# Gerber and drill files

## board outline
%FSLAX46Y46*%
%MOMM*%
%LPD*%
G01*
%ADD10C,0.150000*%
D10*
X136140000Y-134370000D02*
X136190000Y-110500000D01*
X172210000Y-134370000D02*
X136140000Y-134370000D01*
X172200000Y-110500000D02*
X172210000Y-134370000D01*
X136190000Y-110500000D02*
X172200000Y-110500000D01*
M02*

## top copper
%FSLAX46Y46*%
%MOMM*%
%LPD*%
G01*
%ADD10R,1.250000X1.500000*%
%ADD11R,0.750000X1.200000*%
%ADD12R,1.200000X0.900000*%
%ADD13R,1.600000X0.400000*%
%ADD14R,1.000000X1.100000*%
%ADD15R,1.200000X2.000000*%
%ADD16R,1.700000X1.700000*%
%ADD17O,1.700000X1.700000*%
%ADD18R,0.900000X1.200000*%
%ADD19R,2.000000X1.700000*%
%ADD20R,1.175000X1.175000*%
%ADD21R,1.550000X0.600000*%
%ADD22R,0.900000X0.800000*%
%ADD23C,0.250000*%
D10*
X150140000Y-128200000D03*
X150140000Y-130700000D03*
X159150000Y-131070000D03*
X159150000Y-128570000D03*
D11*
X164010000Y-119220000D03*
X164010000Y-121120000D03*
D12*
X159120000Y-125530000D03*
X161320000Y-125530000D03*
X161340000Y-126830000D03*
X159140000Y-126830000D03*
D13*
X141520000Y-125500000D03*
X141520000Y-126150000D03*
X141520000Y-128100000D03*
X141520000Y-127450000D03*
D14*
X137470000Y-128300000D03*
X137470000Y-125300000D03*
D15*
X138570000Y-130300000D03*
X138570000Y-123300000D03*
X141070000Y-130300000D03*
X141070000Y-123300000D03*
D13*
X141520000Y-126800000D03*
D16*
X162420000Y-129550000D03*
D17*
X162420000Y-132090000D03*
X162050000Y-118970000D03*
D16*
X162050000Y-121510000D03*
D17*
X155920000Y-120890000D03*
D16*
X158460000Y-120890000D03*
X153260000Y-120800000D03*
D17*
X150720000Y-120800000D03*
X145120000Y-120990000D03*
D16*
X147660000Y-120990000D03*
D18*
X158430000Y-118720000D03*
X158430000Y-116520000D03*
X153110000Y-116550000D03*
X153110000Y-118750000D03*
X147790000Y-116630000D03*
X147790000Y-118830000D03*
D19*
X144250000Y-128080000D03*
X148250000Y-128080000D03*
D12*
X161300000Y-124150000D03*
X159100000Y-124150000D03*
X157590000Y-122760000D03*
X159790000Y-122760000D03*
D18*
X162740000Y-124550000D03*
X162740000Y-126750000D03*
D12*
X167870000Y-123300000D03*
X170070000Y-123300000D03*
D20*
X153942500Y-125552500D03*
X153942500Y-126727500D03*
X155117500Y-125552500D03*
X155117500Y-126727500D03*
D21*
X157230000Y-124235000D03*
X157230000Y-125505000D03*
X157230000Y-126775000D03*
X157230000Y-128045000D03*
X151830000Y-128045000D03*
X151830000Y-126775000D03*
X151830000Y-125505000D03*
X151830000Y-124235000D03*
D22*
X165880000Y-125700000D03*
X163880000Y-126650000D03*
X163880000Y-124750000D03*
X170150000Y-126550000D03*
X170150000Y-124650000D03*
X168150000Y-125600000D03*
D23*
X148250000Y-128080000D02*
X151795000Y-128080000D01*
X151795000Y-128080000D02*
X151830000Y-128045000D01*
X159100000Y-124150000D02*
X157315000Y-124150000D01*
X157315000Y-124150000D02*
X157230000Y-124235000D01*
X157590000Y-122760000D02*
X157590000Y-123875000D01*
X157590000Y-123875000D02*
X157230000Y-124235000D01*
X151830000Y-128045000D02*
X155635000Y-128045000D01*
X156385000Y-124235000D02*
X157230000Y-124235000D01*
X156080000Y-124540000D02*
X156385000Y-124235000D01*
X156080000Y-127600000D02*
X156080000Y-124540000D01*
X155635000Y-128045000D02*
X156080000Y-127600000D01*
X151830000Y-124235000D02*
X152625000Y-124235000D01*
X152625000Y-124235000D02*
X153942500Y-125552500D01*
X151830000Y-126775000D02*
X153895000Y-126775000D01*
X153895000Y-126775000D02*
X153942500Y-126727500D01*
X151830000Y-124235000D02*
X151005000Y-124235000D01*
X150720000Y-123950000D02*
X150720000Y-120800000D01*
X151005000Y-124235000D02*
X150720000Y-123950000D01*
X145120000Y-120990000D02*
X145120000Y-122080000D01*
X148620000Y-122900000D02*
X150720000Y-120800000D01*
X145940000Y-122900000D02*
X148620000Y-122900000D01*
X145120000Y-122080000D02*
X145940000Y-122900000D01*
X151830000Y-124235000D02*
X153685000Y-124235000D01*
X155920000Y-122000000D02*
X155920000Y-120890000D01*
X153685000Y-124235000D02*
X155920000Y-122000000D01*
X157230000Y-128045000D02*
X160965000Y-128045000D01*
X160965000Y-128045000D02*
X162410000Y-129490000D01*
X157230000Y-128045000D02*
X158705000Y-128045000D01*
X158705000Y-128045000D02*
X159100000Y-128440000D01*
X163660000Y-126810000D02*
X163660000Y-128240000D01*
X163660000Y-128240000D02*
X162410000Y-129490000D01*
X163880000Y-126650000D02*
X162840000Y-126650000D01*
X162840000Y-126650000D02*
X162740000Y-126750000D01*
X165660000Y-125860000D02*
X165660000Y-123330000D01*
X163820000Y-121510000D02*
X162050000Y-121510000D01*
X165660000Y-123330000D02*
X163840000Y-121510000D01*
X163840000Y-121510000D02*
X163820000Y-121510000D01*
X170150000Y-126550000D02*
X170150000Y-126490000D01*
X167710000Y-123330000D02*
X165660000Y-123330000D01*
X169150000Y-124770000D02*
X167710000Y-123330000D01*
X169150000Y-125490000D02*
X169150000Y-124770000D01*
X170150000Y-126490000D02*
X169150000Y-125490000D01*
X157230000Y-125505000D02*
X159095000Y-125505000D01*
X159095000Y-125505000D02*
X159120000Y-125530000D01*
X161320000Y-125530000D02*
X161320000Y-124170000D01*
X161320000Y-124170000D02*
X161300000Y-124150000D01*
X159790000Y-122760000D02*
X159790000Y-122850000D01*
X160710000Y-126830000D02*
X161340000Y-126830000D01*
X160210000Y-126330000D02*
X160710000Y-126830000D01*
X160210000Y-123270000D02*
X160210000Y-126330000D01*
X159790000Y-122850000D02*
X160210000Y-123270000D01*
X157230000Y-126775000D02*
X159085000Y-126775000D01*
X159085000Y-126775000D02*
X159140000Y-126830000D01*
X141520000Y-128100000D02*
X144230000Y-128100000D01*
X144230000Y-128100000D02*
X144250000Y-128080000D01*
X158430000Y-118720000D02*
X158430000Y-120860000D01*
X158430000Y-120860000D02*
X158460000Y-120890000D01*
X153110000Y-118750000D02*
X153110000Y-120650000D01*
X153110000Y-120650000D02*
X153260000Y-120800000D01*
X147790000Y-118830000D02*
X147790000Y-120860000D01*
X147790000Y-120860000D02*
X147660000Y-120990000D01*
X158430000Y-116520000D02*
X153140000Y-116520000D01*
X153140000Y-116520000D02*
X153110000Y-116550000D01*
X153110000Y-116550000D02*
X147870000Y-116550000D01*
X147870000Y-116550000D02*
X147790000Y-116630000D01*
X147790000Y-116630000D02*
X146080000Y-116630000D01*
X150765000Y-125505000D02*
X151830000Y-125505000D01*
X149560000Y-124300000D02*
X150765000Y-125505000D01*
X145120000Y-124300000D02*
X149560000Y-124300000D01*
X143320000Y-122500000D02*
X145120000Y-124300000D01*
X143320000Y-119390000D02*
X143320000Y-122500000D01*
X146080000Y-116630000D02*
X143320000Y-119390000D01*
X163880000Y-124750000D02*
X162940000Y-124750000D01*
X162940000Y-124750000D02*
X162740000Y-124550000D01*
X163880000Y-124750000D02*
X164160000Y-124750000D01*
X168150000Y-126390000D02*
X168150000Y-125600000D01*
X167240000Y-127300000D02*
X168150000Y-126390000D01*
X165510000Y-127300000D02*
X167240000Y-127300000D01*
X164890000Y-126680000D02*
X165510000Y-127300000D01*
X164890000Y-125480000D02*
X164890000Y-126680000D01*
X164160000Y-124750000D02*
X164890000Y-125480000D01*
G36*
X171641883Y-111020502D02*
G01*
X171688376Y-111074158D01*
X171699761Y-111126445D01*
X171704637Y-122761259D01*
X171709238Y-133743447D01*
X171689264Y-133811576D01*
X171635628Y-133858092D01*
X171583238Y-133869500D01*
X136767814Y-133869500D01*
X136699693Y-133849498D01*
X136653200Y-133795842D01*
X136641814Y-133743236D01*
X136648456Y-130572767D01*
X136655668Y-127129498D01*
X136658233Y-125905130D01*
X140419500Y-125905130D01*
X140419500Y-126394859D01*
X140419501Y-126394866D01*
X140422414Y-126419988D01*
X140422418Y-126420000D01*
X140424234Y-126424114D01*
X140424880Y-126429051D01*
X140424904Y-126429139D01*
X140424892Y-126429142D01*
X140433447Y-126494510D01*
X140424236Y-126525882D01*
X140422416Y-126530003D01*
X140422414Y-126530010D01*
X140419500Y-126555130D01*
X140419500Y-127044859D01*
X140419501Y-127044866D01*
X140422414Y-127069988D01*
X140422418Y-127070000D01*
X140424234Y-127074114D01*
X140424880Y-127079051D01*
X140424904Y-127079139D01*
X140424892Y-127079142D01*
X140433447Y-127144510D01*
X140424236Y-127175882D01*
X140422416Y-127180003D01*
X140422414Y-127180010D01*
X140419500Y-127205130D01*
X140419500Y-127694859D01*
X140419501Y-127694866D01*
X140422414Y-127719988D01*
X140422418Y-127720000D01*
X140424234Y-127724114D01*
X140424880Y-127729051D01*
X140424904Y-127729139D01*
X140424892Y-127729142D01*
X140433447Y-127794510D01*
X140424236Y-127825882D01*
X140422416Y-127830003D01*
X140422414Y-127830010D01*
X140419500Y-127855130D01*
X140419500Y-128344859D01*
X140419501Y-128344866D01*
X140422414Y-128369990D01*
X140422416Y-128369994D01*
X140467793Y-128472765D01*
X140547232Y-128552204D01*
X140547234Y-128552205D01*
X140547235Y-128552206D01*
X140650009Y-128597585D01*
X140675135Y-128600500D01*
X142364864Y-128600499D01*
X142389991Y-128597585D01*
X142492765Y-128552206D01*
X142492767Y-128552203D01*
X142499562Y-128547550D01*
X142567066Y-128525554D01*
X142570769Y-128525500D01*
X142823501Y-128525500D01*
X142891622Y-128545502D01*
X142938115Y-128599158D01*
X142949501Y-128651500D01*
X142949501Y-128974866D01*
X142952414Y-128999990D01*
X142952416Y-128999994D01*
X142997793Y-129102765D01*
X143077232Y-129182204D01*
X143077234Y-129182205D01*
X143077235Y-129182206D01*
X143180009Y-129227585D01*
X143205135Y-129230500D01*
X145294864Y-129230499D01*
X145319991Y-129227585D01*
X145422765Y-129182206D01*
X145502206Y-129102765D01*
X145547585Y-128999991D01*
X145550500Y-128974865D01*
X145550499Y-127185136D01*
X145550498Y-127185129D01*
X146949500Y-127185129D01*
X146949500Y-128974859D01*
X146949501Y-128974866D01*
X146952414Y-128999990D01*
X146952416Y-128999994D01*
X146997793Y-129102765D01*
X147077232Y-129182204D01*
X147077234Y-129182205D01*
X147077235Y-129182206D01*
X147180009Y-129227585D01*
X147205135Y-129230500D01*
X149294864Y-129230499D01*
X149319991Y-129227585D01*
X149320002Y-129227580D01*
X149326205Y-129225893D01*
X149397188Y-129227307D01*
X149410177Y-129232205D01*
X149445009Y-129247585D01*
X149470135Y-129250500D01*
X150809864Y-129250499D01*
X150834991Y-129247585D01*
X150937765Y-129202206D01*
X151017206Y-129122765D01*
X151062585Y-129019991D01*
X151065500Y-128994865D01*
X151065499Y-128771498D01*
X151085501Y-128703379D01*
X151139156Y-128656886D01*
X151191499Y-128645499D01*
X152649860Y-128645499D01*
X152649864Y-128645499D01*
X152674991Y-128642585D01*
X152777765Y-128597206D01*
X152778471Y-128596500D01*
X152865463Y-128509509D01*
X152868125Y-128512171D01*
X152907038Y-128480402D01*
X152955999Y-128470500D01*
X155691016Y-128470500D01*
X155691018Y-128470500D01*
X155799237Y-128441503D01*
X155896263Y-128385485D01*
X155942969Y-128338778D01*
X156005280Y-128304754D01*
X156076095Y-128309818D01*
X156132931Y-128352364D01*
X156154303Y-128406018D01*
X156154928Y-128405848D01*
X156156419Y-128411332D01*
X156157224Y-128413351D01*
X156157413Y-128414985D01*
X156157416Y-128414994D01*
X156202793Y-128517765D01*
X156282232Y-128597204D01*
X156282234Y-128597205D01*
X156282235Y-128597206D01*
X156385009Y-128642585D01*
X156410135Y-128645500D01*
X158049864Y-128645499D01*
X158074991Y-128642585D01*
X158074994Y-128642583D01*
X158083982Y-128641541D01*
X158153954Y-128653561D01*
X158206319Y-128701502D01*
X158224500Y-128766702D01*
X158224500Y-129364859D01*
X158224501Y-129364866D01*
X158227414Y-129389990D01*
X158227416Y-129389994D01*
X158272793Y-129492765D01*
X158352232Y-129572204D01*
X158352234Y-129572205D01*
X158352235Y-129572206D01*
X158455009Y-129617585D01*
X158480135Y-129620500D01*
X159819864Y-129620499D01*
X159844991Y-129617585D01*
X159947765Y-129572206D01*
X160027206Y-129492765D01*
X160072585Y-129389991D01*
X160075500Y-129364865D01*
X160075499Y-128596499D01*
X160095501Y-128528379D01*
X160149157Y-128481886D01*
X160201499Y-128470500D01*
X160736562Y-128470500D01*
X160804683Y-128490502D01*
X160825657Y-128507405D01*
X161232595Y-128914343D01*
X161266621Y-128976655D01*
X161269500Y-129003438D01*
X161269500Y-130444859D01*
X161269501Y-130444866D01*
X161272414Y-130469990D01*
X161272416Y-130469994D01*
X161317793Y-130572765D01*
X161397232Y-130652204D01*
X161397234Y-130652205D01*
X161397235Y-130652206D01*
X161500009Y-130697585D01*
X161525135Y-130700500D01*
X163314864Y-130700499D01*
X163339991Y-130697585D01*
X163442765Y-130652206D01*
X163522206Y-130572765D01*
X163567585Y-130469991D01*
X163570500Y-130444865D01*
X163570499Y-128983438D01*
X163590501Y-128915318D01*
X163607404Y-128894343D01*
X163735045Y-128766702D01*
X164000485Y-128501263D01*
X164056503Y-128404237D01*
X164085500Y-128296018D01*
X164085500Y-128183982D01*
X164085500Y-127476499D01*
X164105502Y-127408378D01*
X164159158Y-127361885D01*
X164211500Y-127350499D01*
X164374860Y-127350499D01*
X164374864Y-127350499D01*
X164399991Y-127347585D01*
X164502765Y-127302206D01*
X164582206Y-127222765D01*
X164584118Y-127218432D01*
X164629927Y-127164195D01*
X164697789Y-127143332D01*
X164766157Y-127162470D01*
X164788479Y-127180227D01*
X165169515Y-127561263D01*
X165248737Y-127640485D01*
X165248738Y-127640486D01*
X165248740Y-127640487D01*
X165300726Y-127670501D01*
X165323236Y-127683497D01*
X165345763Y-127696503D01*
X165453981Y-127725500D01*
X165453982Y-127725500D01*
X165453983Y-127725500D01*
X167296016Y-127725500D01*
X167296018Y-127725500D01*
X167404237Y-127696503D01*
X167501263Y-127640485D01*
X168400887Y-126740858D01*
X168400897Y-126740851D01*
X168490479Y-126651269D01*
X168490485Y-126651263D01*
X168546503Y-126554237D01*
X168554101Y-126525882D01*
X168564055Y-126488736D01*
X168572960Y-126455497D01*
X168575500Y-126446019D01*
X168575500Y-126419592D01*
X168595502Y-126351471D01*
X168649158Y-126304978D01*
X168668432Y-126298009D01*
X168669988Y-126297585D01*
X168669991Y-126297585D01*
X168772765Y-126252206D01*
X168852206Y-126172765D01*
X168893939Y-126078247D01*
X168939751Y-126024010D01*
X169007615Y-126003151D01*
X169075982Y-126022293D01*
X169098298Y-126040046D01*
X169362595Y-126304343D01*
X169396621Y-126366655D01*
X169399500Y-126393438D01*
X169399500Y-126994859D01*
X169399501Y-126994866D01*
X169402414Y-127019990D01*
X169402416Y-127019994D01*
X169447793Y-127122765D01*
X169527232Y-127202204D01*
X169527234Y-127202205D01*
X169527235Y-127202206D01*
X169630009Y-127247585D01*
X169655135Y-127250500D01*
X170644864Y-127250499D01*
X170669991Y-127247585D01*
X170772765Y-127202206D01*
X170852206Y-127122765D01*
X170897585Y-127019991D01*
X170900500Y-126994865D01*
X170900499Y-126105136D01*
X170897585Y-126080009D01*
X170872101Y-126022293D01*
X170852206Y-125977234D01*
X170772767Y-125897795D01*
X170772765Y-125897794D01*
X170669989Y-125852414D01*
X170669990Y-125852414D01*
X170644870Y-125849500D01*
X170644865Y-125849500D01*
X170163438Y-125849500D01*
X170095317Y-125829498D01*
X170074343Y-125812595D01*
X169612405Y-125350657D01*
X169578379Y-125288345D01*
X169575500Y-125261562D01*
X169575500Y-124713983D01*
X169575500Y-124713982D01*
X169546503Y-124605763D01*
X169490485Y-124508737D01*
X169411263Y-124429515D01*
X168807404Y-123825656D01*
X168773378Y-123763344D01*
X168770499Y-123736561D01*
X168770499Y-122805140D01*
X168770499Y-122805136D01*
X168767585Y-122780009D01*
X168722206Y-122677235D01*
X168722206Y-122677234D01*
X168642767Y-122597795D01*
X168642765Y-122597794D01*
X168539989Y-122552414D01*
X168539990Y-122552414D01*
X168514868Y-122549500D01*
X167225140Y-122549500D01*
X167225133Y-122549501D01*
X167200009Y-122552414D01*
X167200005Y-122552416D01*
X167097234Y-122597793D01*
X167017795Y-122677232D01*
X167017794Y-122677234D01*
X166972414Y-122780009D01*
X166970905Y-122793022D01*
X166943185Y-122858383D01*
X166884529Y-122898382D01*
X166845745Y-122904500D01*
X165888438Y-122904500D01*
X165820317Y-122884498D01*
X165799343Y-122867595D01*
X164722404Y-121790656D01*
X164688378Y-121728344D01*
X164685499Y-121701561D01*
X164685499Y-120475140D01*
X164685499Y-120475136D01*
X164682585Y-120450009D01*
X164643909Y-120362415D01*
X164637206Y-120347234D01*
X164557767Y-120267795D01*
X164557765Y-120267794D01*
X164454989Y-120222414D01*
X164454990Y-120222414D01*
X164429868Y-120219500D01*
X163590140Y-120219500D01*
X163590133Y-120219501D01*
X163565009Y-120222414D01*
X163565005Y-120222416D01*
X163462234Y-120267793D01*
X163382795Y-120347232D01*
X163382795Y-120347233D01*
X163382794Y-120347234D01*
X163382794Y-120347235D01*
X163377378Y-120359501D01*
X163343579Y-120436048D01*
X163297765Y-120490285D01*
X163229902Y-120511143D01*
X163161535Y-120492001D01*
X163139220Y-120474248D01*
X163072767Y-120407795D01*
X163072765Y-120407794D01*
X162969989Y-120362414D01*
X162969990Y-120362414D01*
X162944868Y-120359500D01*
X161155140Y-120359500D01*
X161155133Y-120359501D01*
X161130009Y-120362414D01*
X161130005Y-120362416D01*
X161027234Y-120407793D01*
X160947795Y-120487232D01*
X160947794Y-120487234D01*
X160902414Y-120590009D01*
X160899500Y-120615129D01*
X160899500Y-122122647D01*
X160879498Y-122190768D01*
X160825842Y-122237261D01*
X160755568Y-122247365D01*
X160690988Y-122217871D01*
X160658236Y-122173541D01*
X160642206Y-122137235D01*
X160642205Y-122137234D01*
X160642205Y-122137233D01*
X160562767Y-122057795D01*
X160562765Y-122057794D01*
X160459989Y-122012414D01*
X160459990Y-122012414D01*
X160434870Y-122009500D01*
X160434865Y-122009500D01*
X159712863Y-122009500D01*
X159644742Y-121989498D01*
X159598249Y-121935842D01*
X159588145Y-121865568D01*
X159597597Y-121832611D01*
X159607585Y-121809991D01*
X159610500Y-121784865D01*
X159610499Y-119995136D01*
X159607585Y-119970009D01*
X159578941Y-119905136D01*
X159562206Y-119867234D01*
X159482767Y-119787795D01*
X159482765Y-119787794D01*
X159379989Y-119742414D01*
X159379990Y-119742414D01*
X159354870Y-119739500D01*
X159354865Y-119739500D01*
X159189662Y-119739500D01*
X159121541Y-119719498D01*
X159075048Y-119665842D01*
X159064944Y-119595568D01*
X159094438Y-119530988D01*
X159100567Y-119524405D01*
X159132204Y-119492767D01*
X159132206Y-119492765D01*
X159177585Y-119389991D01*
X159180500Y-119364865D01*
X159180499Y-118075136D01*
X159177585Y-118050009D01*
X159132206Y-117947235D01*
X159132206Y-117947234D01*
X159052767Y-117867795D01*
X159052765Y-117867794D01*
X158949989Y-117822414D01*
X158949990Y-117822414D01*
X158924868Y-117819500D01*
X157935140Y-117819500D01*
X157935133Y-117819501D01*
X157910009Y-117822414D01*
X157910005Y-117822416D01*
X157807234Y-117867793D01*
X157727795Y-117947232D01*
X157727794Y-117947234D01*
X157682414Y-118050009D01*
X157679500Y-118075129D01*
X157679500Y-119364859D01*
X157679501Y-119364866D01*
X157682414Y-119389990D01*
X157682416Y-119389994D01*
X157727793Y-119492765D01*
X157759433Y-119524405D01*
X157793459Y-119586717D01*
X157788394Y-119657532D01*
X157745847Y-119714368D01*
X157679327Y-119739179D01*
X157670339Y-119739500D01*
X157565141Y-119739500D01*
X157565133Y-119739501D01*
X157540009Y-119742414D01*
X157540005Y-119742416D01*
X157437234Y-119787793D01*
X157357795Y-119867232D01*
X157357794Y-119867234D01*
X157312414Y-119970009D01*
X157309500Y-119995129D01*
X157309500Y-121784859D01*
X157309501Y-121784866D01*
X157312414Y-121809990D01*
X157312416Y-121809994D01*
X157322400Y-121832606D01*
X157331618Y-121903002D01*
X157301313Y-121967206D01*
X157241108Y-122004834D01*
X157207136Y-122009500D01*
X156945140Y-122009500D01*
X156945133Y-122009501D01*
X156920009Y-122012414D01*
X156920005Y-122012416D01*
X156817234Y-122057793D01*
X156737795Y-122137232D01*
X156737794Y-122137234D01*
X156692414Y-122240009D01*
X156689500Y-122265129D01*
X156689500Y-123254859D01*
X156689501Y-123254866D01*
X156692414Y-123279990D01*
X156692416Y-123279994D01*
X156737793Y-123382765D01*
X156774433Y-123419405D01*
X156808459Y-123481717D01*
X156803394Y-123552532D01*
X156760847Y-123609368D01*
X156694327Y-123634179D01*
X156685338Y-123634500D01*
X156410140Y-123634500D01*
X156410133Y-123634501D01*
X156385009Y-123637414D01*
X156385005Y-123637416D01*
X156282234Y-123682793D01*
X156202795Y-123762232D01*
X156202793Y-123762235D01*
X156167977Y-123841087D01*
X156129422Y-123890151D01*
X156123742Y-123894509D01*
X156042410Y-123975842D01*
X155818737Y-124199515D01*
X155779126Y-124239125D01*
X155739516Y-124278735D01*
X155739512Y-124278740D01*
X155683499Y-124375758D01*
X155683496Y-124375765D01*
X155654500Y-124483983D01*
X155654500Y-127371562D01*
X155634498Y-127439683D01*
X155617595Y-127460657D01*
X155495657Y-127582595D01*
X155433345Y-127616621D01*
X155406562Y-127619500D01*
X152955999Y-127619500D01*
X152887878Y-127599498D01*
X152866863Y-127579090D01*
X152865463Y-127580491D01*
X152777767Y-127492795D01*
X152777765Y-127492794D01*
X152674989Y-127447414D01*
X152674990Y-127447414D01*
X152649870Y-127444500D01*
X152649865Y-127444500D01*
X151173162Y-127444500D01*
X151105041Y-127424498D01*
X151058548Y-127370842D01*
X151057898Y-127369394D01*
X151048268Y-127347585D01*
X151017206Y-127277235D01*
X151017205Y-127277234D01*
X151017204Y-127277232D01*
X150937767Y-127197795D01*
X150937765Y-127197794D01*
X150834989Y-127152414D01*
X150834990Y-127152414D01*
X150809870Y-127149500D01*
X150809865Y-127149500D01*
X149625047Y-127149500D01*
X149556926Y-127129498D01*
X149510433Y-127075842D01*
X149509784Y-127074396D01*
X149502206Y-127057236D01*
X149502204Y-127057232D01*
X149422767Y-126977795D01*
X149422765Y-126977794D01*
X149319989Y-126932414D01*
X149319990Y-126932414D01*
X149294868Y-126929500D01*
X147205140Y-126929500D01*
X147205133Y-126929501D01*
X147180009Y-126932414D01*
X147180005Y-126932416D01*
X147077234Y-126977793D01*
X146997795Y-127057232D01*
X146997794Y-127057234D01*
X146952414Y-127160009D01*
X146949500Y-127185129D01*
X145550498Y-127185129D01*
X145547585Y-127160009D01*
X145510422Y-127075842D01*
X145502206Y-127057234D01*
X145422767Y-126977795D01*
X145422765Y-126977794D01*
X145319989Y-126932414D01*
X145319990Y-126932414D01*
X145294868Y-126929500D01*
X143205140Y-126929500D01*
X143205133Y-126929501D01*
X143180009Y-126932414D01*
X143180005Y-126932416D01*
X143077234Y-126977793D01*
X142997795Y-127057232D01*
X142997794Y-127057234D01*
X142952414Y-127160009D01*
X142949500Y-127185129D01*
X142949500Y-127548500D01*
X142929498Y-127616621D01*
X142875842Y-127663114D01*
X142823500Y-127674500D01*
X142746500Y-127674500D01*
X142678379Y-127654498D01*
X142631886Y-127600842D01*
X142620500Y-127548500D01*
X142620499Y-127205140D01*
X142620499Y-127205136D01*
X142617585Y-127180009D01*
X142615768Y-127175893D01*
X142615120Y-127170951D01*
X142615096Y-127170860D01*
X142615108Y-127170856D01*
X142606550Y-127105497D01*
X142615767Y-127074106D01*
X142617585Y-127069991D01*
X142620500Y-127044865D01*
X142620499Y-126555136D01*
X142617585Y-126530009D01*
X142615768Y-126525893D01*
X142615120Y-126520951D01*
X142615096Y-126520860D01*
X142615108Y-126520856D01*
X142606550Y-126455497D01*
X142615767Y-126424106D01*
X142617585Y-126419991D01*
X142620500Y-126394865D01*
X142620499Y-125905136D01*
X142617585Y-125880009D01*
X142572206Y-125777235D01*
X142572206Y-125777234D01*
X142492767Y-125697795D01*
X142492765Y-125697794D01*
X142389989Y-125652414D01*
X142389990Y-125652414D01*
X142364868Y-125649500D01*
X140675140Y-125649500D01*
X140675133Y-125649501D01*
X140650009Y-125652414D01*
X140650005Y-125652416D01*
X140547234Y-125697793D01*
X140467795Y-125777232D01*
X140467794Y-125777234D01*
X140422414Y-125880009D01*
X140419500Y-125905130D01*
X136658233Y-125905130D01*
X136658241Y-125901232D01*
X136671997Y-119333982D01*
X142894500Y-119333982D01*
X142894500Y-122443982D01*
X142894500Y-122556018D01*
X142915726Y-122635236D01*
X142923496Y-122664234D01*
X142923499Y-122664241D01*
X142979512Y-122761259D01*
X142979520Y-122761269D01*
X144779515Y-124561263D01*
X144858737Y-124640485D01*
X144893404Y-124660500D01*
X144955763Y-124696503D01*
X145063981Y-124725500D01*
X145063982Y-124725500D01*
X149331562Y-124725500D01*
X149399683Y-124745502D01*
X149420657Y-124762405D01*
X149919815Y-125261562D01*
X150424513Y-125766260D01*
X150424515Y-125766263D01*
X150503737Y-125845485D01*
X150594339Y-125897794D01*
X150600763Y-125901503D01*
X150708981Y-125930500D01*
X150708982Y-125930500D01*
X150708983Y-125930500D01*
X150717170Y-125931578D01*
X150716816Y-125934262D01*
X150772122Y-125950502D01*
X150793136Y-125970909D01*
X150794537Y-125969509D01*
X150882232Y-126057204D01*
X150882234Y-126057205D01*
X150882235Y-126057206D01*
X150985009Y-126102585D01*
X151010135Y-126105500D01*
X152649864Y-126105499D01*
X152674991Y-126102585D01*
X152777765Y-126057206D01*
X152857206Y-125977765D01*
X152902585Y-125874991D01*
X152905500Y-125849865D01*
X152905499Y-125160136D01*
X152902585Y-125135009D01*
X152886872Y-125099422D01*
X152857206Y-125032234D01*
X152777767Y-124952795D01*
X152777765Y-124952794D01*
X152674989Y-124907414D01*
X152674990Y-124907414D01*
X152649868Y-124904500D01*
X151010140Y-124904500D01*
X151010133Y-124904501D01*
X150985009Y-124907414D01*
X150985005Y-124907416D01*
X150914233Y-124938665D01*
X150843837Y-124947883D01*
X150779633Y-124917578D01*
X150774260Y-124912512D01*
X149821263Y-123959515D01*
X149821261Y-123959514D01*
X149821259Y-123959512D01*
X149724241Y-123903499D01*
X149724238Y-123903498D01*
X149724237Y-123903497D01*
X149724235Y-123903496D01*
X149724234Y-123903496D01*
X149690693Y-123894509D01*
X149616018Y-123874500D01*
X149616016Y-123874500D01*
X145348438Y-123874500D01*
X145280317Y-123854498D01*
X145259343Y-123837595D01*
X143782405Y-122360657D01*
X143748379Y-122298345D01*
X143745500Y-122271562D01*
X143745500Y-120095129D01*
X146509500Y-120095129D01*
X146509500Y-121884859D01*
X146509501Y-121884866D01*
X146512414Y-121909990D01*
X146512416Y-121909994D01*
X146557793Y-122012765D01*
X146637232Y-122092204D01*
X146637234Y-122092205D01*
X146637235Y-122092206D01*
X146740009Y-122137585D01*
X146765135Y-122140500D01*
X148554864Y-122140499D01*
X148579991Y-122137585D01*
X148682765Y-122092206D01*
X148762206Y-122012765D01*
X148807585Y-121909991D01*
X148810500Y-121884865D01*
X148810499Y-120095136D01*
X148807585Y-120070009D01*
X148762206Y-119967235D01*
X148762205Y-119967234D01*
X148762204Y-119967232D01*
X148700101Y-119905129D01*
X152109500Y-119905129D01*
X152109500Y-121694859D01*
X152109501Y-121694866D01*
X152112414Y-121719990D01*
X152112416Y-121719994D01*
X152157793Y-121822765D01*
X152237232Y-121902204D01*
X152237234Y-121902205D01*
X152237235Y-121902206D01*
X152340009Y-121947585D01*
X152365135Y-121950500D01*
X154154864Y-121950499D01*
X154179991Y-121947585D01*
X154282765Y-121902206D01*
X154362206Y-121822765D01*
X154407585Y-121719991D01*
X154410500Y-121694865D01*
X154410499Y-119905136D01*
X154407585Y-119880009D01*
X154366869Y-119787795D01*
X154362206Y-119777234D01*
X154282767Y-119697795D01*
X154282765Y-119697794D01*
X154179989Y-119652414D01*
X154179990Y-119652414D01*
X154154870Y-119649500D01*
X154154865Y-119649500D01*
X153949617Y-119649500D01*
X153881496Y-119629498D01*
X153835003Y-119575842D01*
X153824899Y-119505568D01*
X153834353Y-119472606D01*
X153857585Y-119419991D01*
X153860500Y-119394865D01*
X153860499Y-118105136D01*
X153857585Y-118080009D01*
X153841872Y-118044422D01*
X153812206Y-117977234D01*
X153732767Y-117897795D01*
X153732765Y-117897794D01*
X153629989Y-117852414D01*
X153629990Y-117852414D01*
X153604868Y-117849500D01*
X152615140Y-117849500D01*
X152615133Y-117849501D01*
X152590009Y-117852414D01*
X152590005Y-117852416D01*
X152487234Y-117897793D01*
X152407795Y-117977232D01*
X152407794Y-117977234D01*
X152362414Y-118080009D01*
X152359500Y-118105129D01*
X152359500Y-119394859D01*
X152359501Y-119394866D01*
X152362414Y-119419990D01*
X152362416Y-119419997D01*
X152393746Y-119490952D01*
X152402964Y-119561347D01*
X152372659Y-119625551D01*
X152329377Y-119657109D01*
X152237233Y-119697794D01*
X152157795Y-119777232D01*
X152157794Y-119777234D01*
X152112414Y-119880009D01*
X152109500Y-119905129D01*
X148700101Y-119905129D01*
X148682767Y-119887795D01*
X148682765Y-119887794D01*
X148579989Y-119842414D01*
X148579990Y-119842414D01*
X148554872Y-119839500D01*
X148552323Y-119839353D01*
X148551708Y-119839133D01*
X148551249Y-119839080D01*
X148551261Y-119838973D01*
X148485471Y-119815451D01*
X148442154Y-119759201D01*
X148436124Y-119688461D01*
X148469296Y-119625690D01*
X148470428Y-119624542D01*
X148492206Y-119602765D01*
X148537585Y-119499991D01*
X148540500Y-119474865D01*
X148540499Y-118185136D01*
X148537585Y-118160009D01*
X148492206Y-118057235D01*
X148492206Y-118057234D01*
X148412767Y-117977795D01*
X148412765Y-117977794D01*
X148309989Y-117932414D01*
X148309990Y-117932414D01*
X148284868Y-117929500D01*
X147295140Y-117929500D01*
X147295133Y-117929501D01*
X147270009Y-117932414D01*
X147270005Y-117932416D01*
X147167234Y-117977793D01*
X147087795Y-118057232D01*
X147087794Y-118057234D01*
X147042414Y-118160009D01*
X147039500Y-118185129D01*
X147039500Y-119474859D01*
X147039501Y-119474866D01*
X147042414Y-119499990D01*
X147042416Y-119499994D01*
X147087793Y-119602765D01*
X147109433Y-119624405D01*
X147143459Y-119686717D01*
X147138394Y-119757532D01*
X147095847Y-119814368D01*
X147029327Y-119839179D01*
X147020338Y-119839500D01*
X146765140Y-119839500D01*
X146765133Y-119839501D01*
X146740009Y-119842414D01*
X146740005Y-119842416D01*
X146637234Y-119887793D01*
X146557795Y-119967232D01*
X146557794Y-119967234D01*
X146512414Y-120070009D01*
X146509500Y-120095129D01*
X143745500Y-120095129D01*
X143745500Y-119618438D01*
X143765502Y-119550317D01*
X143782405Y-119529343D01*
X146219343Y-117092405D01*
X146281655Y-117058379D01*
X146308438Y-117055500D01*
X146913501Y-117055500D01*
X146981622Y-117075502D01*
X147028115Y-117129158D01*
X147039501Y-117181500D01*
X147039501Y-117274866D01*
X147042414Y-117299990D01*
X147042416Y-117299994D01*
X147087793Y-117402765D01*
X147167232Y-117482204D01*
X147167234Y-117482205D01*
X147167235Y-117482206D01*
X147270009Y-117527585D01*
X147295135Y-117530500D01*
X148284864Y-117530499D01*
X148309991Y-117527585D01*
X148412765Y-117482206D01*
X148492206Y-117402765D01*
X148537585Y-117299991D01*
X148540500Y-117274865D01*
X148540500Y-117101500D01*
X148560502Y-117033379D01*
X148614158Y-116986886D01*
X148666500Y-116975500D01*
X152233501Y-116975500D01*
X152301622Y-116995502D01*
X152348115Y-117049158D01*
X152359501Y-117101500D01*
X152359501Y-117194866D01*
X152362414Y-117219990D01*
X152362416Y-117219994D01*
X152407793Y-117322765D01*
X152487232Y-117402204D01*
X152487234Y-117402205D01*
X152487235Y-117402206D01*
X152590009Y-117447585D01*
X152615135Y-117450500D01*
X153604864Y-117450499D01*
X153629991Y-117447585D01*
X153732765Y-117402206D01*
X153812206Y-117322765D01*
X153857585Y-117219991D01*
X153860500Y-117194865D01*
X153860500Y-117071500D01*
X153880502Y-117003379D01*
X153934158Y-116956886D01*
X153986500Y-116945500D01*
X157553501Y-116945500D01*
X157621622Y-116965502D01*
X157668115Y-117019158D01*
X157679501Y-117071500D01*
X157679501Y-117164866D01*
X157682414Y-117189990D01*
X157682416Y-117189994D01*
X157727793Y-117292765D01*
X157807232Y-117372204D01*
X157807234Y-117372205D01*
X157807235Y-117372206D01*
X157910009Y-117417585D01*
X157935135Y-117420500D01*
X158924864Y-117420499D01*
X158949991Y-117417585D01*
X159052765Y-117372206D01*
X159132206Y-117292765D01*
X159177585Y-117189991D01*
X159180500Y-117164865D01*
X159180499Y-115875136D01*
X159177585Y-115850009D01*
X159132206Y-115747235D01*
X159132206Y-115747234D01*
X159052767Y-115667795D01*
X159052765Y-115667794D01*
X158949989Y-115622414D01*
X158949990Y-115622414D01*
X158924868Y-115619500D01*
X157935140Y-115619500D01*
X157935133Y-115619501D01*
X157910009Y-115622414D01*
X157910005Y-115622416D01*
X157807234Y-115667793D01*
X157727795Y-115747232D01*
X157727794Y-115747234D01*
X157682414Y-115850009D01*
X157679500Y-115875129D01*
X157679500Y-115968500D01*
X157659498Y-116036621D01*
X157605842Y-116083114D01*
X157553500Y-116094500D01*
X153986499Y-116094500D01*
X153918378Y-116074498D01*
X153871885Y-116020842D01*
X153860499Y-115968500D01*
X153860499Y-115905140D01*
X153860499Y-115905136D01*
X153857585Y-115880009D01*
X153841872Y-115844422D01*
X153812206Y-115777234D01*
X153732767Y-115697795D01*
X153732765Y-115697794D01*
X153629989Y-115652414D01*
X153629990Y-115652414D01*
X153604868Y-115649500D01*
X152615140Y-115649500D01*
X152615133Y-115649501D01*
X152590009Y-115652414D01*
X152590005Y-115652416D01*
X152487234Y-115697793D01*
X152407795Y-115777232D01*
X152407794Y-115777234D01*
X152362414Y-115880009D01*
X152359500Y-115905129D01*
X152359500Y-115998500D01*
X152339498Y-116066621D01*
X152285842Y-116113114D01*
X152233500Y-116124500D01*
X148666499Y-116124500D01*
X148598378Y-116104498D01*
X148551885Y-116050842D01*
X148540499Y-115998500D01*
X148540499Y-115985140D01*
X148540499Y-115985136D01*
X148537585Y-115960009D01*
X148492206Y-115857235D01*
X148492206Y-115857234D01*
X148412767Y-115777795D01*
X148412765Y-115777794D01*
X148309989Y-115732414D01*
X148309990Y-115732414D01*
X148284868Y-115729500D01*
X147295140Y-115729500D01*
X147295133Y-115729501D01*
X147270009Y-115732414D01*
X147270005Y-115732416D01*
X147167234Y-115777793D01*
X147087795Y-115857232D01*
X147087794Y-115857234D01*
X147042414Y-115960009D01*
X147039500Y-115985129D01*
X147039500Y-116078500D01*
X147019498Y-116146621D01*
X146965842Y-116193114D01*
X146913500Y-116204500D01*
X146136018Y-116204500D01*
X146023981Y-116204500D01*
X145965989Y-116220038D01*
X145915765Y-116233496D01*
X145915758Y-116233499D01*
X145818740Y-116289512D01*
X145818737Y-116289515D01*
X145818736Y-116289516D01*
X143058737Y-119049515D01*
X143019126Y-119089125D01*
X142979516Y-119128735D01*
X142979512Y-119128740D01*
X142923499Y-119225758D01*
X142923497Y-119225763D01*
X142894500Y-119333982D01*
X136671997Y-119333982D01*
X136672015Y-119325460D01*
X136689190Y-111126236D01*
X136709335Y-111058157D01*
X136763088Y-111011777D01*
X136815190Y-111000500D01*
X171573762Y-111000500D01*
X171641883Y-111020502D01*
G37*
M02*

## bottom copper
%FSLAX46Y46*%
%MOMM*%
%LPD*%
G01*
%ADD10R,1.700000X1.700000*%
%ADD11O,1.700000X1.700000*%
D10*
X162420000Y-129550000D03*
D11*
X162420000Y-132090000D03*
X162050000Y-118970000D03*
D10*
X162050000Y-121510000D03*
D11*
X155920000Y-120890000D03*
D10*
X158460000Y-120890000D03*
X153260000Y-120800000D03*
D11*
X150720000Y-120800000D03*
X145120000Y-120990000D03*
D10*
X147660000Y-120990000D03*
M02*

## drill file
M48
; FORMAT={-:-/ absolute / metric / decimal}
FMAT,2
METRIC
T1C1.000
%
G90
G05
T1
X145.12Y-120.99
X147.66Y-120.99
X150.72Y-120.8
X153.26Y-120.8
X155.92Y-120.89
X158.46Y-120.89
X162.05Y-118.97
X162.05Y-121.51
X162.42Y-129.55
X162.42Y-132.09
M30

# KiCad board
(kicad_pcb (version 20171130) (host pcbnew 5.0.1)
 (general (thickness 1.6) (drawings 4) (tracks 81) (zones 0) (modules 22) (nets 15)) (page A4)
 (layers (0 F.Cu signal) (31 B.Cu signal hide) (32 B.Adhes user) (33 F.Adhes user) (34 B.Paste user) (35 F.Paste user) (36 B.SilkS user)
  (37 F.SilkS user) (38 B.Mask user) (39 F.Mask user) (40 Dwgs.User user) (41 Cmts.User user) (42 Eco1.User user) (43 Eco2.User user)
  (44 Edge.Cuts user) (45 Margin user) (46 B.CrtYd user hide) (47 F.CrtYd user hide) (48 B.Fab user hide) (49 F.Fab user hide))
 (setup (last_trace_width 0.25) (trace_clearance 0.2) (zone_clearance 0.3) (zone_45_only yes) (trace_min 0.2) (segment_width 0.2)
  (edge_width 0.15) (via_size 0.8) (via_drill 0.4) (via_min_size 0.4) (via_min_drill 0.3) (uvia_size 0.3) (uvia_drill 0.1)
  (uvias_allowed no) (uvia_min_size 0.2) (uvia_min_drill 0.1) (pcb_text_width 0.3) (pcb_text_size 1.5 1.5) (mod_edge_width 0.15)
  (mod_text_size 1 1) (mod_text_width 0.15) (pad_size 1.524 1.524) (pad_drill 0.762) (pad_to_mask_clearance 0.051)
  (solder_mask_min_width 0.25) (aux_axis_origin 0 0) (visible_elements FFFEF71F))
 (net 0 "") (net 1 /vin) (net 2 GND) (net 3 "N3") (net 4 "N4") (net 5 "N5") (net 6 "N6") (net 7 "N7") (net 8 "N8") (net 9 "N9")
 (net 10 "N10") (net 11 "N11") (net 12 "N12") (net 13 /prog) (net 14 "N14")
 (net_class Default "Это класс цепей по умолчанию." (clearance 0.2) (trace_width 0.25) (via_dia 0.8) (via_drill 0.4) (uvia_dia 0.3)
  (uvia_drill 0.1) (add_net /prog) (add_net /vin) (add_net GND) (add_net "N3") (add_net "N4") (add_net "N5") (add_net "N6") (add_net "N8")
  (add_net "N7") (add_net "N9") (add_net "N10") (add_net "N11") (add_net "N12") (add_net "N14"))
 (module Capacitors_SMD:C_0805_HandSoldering (layer F.Cu) (at 150.14 129.45 270)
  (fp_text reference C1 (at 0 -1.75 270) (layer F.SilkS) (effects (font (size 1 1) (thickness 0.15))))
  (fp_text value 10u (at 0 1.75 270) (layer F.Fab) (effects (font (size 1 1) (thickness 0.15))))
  (pad 1 smd rect (at -1.25 0 270) (size 1.5 1.25) (layers F.Cu F.Paste F.Mask) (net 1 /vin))
  (pad 2 smd rect (at 1.25 0 270) (size 1.5 1.25) (layers F.Cu F.Paste F.Mask) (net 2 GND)))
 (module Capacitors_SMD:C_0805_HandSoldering (layer F.Cu) (at 159.15 129.82 270)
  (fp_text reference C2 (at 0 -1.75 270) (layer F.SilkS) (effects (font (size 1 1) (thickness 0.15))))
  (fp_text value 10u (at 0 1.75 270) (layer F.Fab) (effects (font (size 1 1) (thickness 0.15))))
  (pad 2 smd rect (at 1.25 0 270) (size 1.5 1.25) (layers F.Cu F.Paste F.Mask) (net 2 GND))
  (pad 1 smd rect (at -1.25 0 270) (size 1.5 1.25) (layers F.Cu F.Paste F.Mask) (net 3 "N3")))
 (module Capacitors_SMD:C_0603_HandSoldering (layer F.Cu) (at 164.01 120.17 90)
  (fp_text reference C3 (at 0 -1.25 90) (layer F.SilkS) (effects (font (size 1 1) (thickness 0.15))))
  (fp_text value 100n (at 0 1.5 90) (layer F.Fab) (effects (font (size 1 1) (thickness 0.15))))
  (pad 2 smd rect (at 0.95 0 90) (size 1.2 0.75) (layers F.Cu F.Paste F.Mask) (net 2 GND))
  (pad 1 smd rect (at -0.95 0 90) (size 1.2 0.75) (layers F.Cu F.Paste F.Mask) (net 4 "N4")))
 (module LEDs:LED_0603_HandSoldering (layer F.Cu) (at 160.22 125.53)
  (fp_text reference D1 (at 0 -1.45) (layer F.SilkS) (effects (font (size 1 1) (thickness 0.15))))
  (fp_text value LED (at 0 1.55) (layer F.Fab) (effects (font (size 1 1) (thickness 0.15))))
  (pad 1 smd rect (at -1.1 0) (size 1.2 0.9) (layers F.Cu F.Paste F.Mask) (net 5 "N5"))
  (pad 2 smd rect (at 1.1 0) (size 1.2 0.9) (layers F.Cu F.Paste F.Mask) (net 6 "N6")))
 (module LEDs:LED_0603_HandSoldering (layer F.Cu) (at 160.24 126.83)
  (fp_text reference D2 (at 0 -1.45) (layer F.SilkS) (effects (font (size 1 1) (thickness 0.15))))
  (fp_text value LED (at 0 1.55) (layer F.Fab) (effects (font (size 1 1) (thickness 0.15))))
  (pad 2 smd rect (at 1.1 0) (size 1.2 0.9) (layers F.Cu F.Paste F.Mask) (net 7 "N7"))
  (pad 1 smd rect (at -1.1 0) (size 1.2 0.9) (layers F.Cu F.Paste F.Mask) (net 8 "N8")))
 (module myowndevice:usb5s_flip (layer F.Cu) (at 142.42 126.8 270)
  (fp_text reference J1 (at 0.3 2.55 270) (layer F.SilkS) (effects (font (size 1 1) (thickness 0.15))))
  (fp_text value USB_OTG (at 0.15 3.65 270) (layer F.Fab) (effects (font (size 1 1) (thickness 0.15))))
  (pad 5 smd rect (at -1.3 0.9 270) (size 0.4 1.6) (layers F.Cu F.Paste F.Mask) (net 2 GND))
  (pad 4 smd rect (at -0.65 0.9 270) (size 0.4 1.6) (layers F.Cu F.Paste F.Mask))
  (pad 1 smd rect (at 1.3 0.9 270) (size 0.4 1.6) (layers F.Cu F.Paste F.Mask) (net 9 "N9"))
  (pad 2 smd rect (at 0.65 0.9 270) (size 0.4 1.6) (layers F.Cu F.Paste F.Mask))
  (pad 5 smd rect (at 1.5 4.95 270) (size 1.1 1) (layers F.Cu F.Paste F.Mask) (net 2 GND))
  (pad 5 smd rect (at -1.5 4.95 270) (size 1.1 1) (layers F.Cu F.Paste F.Mask) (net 2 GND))
  (pad 5 smd rect (at 3.5 3.85 270) (size 2 1.2) (layers F.Cu F.Paste F.Mask) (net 2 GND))
  (pad 5 smd rect (at -3.5 3.85 270) (size 2 1.2) (layers F.Cu F.Paste F.Mask) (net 2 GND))
  (pad 5 smd rect (at 3.5 1.35 270) (size 2 1.2) (layers F.Cu F.Paste F.Mask) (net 2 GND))
  (pad 5 smd rect (at -3.5 1.35 270) (size 2 1.2) (layers F.Cu F.Paste F.Mask) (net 2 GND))
  (pad 3 smd rect (at 0 0.9 270) (size 0.4 1.6) (layers F.Cu F.Paste F.Mask)))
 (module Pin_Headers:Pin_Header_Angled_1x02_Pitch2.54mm (layer B.Cu) (at 162.42 129.55 180)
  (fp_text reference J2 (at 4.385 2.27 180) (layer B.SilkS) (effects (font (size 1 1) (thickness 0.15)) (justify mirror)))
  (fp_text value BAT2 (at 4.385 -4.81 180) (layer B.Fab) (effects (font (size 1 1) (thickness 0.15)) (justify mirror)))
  (pad 1 thru_hole rect (at 0 0 180) (size 1.7 1.7) (drill 1) (layers *.Cu *.Mask) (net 3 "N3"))
  (pad 2 thru_hole oval (at 0 -2.54 180) (size 1.7 1.7) (drill 1) (layers *.Cu *.Mask) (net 2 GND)))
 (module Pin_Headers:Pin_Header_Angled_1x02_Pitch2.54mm (layer B.Cu) (at 162.05 121.51)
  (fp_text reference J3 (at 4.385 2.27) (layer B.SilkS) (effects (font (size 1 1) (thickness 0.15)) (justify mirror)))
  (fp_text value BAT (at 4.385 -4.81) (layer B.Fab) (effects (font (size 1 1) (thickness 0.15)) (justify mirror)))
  (pad 2 thru_hole oval (at 0 -2.54) (size 1.7 1.7) (drill 1) (layers *.Cu *.Mask) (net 2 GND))
  (pad 1 thru_hole rect (at 0 0) (size 1.7 1.7) (drill 1) (layers *.Cu *.Mask) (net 4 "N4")))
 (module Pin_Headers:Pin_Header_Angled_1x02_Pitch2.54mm (layer B.Cu) (at 158.46 120.89 90)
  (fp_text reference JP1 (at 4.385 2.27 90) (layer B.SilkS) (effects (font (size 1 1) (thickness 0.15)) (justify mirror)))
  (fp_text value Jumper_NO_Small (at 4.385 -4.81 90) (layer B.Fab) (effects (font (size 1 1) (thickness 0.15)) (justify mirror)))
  (pad 2 thru_hole oval (at 0 -2.54 90) (size 1.7 1.7) (drill 1) (layers *.Cu *.Mask) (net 2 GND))
  (pad 1 thru_hole rect (at 0 0 90) (size 1.7 1.7) (drill 1) (layers *.Cu *.Mask) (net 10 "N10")))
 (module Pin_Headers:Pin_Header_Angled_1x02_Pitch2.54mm (layer B.Cu) (at 153.26 120.8 90)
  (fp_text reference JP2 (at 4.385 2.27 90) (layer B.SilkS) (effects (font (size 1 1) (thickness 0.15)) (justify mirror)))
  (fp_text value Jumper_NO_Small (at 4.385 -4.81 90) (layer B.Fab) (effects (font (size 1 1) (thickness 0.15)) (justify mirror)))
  (pad 1 thru_hole rect (at 0 0 90) (size 1.7 1.7) (drill 1) (layers *.Cu *.Mask) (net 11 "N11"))
  (pad 2 thru_hole oval (at 0 -2.54 90) (size 1.7 1.7) (drill 1) (layers *.Cu *.Mask) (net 2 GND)))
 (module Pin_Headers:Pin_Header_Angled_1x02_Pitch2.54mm (layer B.Cu) (at 147.66 120.99 90)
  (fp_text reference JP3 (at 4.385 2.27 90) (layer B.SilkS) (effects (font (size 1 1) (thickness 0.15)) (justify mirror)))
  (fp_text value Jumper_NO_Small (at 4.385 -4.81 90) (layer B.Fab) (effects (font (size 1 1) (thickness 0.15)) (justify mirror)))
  (pad 2 thru_hole oval (at 0 -2.54 90) (size 1.7 1.7) (drill 1) (layers *.Cu *.Mask) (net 2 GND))
  (pad 1 thru_hole rect (at 0 0 90) (size 1.7 1.7) (drill 1) (layers *.Cu *.Mask) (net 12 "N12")))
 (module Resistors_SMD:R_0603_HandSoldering (layer F.Cu) (at 158.43 117.62 90)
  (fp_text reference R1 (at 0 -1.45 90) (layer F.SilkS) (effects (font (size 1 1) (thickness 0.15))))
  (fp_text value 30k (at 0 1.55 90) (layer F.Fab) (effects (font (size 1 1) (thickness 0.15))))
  (pad 1 smd rect (at -1.1 0 90) (size 1.2 0.9) (layers F.Cu F.Paste F.Mask) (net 10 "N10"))
  (pad 2 smd rect (at 1.1 0 90) (size 1.2 0.9) (layers F.Cu F.Paste F.Mask) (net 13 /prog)))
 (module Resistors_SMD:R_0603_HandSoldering (layer F.Cu) (at 153.11 117.65 90)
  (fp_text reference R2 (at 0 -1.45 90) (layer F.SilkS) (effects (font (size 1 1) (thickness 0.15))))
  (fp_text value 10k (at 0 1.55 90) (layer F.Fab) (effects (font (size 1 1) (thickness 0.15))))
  (pad 2 smd rect (at 1.1 0 90) (size 1.2 0.9) (layers F.Cu F.Paste F.Mask) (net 13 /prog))
  (pad 1 smd rect (at -1.1 0 90) (size 1.2 0.9) (layers F.Cu F.Paste F.Mask) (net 11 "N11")))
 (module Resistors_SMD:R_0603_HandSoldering (layer F.Cu) (at 147.79 117.73 90)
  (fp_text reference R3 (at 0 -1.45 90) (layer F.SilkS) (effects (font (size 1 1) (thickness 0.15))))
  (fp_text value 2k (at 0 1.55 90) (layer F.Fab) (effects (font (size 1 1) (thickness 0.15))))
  (pad 2 smd rect (at 1.1 0 90) (size 1.2 0.9) (layers F.Cu F.Paste F.Mask) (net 13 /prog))
  (pad 1 smd rect (at -1.1 0 90) (size 1.2 0.9) (layers F.Cu F.Paste F.Mask) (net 12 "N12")))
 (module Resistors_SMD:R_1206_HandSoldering (layer F.Cu) (at 146.25 128.08 180)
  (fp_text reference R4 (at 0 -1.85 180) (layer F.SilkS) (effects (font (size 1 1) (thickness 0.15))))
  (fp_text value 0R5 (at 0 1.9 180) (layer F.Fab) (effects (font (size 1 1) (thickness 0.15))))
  (pad 2 smd rect (at 2 0 180) (size 2 1.7) (layers F.Cu F.Paste F.Mask) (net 9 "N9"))
  (pad 1 smd rect (at -2 0 180) (size 2 1.7) (layers F.Cu F.Paste F.Mask) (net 1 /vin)))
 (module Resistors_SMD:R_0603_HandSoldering (layer F.Cu) (at 160.2 124.15)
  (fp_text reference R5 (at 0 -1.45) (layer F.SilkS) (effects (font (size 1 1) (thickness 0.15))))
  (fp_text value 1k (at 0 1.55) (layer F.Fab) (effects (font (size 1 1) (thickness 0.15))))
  (pad 2 smd rect (at 1.1 0) (size 1.2 0.9) (layers F.Cu F.Paste F.Mask) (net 6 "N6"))
  (pad 1 smd rect (at -1.1 0) (size 1.2 0.9) (layers F.Cu F.Paste F.Mask) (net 1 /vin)))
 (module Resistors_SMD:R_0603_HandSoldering (layer F.Cu) (at 158.69 122.76)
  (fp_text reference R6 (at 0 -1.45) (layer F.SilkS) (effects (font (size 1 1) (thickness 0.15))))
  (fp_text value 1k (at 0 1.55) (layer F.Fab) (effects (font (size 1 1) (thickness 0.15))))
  (pad 1 smd rect (at -1.1 0) (size 1.2 0.9) (layers F.Cu F.Paste F.Mask) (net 1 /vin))
  (pad 2 smd rect (at 1.1 0) (size 1.2 0.9) (layers F.Cu F.Paste F.Mask) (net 7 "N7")))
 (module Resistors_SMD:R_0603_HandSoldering (layer F.Cu) (at 162.74 125.65 270)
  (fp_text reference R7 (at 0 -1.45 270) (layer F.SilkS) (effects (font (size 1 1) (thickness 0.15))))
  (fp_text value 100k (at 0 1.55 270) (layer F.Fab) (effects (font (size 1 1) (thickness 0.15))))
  (pad 1 smd rect (at -1.1 0 270) (size 1.2 0.9) (layers F.Cu F.Paste F.Mask) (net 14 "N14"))
  (pad 2 smd rect (at 1.1 0 270) (size 1.2 0.9) (layers F.Cu F.Paste F.Mask) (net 3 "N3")))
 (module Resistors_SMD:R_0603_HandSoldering (layer F.Cu) (at 168.97 123.3 180)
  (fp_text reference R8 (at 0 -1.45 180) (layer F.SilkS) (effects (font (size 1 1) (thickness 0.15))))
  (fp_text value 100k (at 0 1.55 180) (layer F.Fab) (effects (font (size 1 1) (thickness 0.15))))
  (pad 2 smd rect (at 1.1 0 180) (size 1.2 0.9) (layers F.Cu F.Paste F.Mask) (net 4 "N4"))
  (pad 1 smd rect (at -1.1 0 180) (size 1.2 0.9) (layers F.Cu F.Paste F.Mask) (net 2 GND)))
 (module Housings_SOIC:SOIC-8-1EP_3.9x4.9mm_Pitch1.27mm (layer F.Cu) (at 154.53 126.14)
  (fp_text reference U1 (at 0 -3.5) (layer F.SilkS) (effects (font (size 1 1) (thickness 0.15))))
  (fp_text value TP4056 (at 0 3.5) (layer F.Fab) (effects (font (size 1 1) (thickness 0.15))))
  (pad 9 smd rect (at -0.5875 -0.5875) (size 1.175 1.175) (layers F.Cu F.Paste F.Mask) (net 2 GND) (solder_paste_margin_ratio -0.2))
  (pad 9 smd rect (at -0.5875 0.5875) (size 1.175 1.175) (layers F.Cu F.Paste F.Mask) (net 2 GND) (solder_paste_margin_ratio -0.2))
  (pad 9 smd rect (at 0.5875 -0.5875) (size 1.175 1.175) (layers F.Cu F.Paste F.Mask) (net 2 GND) (solder_paste_margin_ratio -0.2))
  (pad 9 smd rect (at 0.5875 0.5875) (size 1.175 1.175) (layers F.Cu F.Paste F.Mask) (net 2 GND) (solder_paste_margin_ratio -0.2))
  (pad 8 smd rect (at 2.7 -1.905) (size 1.55 0.6) (layers F.Cu F.Paste F.Mask) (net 1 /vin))
  (pad 7 smd rect (at 2.7 -0.635) (size 1.55 0.6) (layers F.Cu F.Paste F.Mask) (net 5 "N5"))
  (pad 6 smd rect (at 2.7 0.635) (size 1.55 0.6) (layers F.Cu F.Paste F.Mask) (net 8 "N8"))
  (pad 5 smd rect (at 2.7 1.905) (size 1.55 0.6) (layers F.Cu F.Paste F.Mask) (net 3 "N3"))
  (pad 4 smd rect (at -2.7 1.905) (size 1.55 0.6) (layers F.Cu F.Paste F.Mask) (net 1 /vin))
  (pad 3 smd rect (at -2.7 0.635) (size 1.55 0.6) (layers F.Cu F.Paste F.Mask) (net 2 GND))
  (pad 2 smd rect (at -2.7 -0.635) (size 1.55 0.6) (layers F.Cu F.Paste F.Mask) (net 13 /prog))
  (pad 1 smd rect (at -2.7 -1.905) (size 1.55 0.6) (layers F.Cu F.Paste F.Mask) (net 2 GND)))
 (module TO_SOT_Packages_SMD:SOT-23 (layer F.Cu) (at 164.88 125.7)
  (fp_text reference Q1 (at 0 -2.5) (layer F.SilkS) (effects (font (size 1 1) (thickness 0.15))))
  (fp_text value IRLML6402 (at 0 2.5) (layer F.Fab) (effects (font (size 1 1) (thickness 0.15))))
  (pad 3 smd rect (at 1 0) (size 0.9 0.8) (layers F.Cu F.Paste F.Mask) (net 4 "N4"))
  (pad 2 smd rect (at -1 0.95) (size 0.9 0.8) (layers F.Cu F.Paste F.Mask) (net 3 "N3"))
  (pad 1 smd rect (at -1 -0.95) (size 0.9 0.8) (layers F.Cu F.Paste F.Mask) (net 14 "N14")))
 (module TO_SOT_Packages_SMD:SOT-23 (layer F.Cu) (at 169.15 125.6 180)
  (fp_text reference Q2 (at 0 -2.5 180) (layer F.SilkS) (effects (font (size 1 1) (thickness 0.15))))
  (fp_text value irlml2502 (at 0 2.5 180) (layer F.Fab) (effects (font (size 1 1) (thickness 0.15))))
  (pad 1 smd rect (at -1 -0.95 180) (size 0.9 0.8) (layers F.Cu F.Paste F.Mask) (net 4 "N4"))
  (pad 2 smd rect (at -1 0.95 180) (size 0.9 0.8) (layers F.Cu F.Paste F.Mask) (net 2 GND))
  (pad 3 smd rect (at 1 0 180) (size 0.9 0.8) (layers F.Cu F.Paste F.Mask) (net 14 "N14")))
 (gr_line (start 136.14 134.37) (end 136.19 110.5) (angle 90) (layer Edge.Cuts) (width 0.15))
 (gr_line (start 172.21 134.37) (end 136.14 134.37) (angle 90) (layer Edge.Cuts) (width 0.15))
 (gr_line (start 172.2 110.5) (end 172.21 134.37) (angle 90) (layer Edge.Cuts) (width 0.15))
 (gr_line (start 136.19 110.5) (end 172.2 110.5) (angle 90) (layer Edge.Cuts) (width 0.15))
 (segment (start 148.25 128.08) (end 151.795 128.08) (width 0.25) (layer F.Cu) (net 1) (status C00000))
 (segment (start 151.795 128.08) (end 151.83 128.045) (width 0.25) (layer F.Cu) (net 1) (status C00000))
 (segment (start 159.1 124.15) (end 157.315 124.15) (width 0.25) (layer F.Cu) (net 1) (status C00000))
 (segment (start 157.315 124.15) (end 157.23 124.235) (width 0.25) (layer F.Cu) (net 1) (status C00000))
 (segment (start 157.59 122.76) (end 157.59 123.875) (width 0.25) (layer F.Cu) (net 1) (status 400000))
 (segment (start 157.59 123.875) (end 157.23 124.235) (width 0.25) (layer F.Cu) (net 1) (status 800000))
 (segment (start 151.83 128.045) (end 155.635 128.045) (width 0.25) (layer F.Cu) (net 1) (status 400000))
 (segment (start 156.385 124.235) (end 157.23 124.235) (width 0.25) (layer F.Cu) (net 1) (status 800000))
 (segment (start 156.08 124.54) (end 156.385 124.235) (width 0.25) (layer F.Cu) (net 1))
 (segment (start 156.08 127.6) (end 156.08 124.54) (width 0.25) (layer F.Cu) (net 1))
 (segment (start 155.635 128.045) (end 156.08 127.6) (width 0.25) (layer F.Cu) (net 1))
 (segment (start 151.83 124.235) (end 152.625 124.235) (width 0.25) (layer F.Cu) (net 2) (status 400000))
 (segment (start 152.625 124.235) (end 153.9425 125.5525) (width 0.25) (layer F.Cu) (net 2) (status 800000))
 (segment (start 151.83 126.775) (end 153.895 126.775) (width 0.25) (layer F.Cu) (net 2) (status C00000))
 (segment (start 153.895 126.775) (end 153.9425 126.7275) (width 0.25) (layer F.Cu) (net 2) (status C00000))
 (segment (start 151.83 124.235) (end 151.005 124.235) (width 0.25) (layer F.Cu) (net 2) (status 400000))
 (segment (start 150.72 123.95) (end 150.72 120.8) (width 0.25) (layer F.Cu) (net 2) (status 800000))
 (segment (start 151.005 124.235) (end 150.72 123.95) (width 0.25) (layer F.Cu) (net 2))
 (segment (start 145.12 120.99) (end 145.12 122.08) (width 0.25) (layer F.Cu) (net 2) (status 400000))
 (segment (start 148.62 122.9) (end 150.72 120.8) (width 0.25) (layer F.Cu) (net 2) (status 800000))
 (segment (start 145.94 122.9) (end 148.62 122.9) (width 0.25) (layer F.Cu) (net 2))
 (segment (start 145.12 122.08) (end 145.94 122.9) (width 0.25) (layer F.Cu) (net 2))
 (segment (start 151.83 124.235) (end 153.685 124.235) (width 0.25) (layer F.Cu) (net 2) (status 400000))
 (segment (start 155.92 122) (end 155.92 120.89) (width 0.25) (layer F.Cu) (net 2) (status 800000))
 (segment (start 153.685 124.235) (end 155.92 122) (width 0.25) (layer F.Cu) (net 2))
 (segment (start 157.23 128.045) (end 160.965 128.045) (width 0.25) (layer F.Cu) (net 3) (status 400000))
 (segment (start 160.965 128.045) (end 162.41 129.49) (width 0.25) (layer F.Cu) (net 3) (status 800000))
 (segment (start 157.23 128.045) (end 158.705 128.045) (width 0.25) (layer F.Cu) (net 3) (status C00000))
 (segment (start 158.705 128.045) (end 159.1 128.44) (width 0.25) (layer F.Cu) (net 3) (status C00000))
 (segment (start 163.66 126.81) (end 163.66 128.24) (width 0.25) (layer F.Cu) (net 3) (status 400000))
 (segment (start 163.66 128.24) (end 162.41 129.49) (width 0.25) (layer F.Cu) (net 3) (status 800000))
 (segment (start 163.88 126.65) (end 162.84 126.65) (width 0.25) (layer F.Cu) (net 3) (status C00000))
 (segment (start 162.84 126.65) (end 162.74 126.75) (width 0.25) (layer F.Cu) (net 3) (status C00000))
 (segment (start 165.66 125.86) (end 165.66 123.33) (width 0.25) (layer F.Cu) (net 4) (status 400000))
 (segment (start 163.82 121.51) (end 162.05 121.51) (width 0.25) (layer F.Cu) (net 4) (status 800000))
 (segment (start 165.66 123.33) (end 163.84 121.51) (width 0.25) (layer F.Cu) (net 4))
 (segment (start 163.84 121.51) (end 163.82 121.51) (width 0.25) (layer F.Cu) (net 4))
 (segment (start 170.15 126.55) (end 170.15 126.49) (width 0.25) (layer F.Cu) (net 4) (status C00000))
 (segment (start 167.71 123.33) (end 165.66 123.33) (width 0.25) (layer F.Cu) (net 4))
 (segment (start 169.15 124.77) (end 167.71 123.33) (width 0.25) (layer F.Cu) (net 4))
 (segment (start 169.15 125.49) (end 169.15 124.77) (width 0.25) (layer F.Cu) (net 4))
 (segment (start 170.15 126.49) (end 169.15 125.49) (width 0.25) (layer F.Cu) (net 4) (status 400000))
 (segment (start 157.23 125.505) (end 159.095 125.505) (width 0.25) (layer F.Cu) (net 5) (status C00000))
 (segment (start 159.095 125.505) (end 159.12 125.53) (width 0.25) (layer F.Cu) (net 5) (status C00000))
 (segment (start 161.32 125.53) (end 161.32 124.17) (width 0.25) (layer F.Cu) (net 6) (status C00000))
 (segment (start 161.32 124.17) (end 161.3 124.15) (width 0.25) (layer F.Cu) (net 6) (status C00000))
 (segment (start 159.79 122.76) (end 159.79 122.85) (width 0.25) (layer F.Cu) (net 7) (status C00000))
 (segment (start 160.71 126.83) (end 161.34 126.83) (width 0.25) (layer F.Cu) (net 7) (status 800000))
 (segment (start 160.21 126.33) (end 160.71 126.83) (width 0.25) (layer F.Cu) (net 7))
 (segment (start 160.21 123.27) (end 160.21 126.33) (width 0.25) (layer F.Cu) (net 7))
 (segment (start 159.79 122.85) (end 160.21 123.27) (width 0.25) (layer F.Cu) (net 7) (status 400000))
 (segment (start 157.23 126.775) (end 159.085 126.775) (width 0.25) (layer F.Cu) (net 8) (status C00000))
 (segment (start 159.085 126.775) (end 159.14 126.83) (width 0.25) (layer F.Cu) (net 8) (status C00000))
 (segment (start 141.52 128.1) (end 144.23 128.1) (width 0.25) (layer F.Cu) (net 9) (status C00000))
 (segment (start 144.23 128.1) (end 144.25 128.08) (width 0.25) (layer F.Cu) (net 9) (status C00000))
 (segment (start 158.43 118.72) (end 158.43 120.86) (width 0.25) (layer F.Cu) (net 10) (status C00000))
 (segment (start 158.43 120.86) (end 158.46 120.89) (width 0.25) (layer F.Cu) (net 10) (status C00000))
 (segment (start 153.11 118.75) (end 153.11 120.65) (width 0.25) (layer F.Cu) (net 11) (status C00000))
 (segment (start 153.11 120.65) (end 153.26 120.8) (width 0.25) (layer F.Cu) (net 11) (status C00000))
 (segment (start 147.79 118.83) (end 147.79 120.86) (width 0.25) (layer F.Cu) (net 12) (status C00000))
 (segment (start 147.79 120.86) (end 147.66 120.99) (width 0.25) (layer F.Cu) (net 12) (status C00000))
 (segment (start 158.43 116.52) (end 153.14 116.52) (width 0.25) (layer F.Cu) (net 13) (status C00000))
 (segment (start 153.14 116.52) (end 153.11 116.55) (width 0.25) (layer F.Cu) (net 13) (status C00000))
 (segment (start 153.11 116.55) (end 147.87 116.55) (width 0.25) (layer F.Cu) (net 13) (status C00000))
 (segment (start 147.87 116.55) (end 147.79 116.63) (width 0.25) (layer F.Cu) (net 13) (status C00000))
 (segment (start 147.79 116.63) (end 146.08 116.63) (width 0.25) (layer F.Cu) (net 13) (status 400000))
 (segment (start 150.765 125.505) (end 151.83 125.505) (width 0.25) (layer F.Cu) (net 13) (status 800000))
 (segment (start 149.56 124.3) (end 150.765 125.505) (width 0.25) (layer F.Cu) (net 13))
 (segment (start 145.12 124.3) (end 149.56 124.3) (width 0.25) (layer F.Cu) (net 13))
 (segment (start 143.32 122.5) (end 145.12 124.3) (width 0.25) (layer F.Cu) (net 13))
 (segment (start 143.32 119.39) (end 143.32 122.5) (width 0.25) (layer F.Cu) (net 13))
 (segment (start 146.08 116.63) (end 143.32 119.39) (width 0.25) (layer F.Cu) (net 13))
 (segment (start 163.88 124.75) (end 162.94 124.75) (width 0.25) (layer F.Cu) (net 14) (status C00000))
 (segment (start 162.94 124.75) (end 162.74 124.55) (width 0.25) (layer F.Cu) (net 14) (status C00000))
 (segment (start 163.88 124.75) (end 164.16 124.75) (width 0.25) (layer F.Cu) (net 14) (status C00000))
 (segment (start 168.15 126.39) (end 168.15 125.6) (width 0.25) (layer F.Cu) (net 14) (status 800000))
 (segment (start 167.24 127.3) (end 168.15 126.39) (width 0.25) (layer F.Cu) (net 14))
 (segment (start 165.51 127.3) (end 167.24 127.3) (width 0.25) (layer F.Cu) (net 14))
 (segment (start 164.89 126.68) (end 165.51 127.3) (width 0.25) (layer F.Cu) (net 14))
 (segment (start 164.89 125.48) (end 164.89 126.68) (width 0.25) (layer F.Cu) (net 14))
 (segment (start 164.16 124.75) (end 164.89 125.48) (width 0.25) (layer F.Cu) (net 14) (status 400000))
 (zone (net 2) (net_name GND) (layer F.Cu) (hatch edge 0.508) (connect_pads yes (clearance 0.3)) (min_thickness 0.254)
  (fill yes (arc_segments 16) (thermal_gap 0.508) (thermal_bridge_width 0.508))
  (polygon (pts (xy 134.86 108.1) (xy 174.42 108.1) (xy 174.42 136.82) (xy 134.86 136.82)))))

